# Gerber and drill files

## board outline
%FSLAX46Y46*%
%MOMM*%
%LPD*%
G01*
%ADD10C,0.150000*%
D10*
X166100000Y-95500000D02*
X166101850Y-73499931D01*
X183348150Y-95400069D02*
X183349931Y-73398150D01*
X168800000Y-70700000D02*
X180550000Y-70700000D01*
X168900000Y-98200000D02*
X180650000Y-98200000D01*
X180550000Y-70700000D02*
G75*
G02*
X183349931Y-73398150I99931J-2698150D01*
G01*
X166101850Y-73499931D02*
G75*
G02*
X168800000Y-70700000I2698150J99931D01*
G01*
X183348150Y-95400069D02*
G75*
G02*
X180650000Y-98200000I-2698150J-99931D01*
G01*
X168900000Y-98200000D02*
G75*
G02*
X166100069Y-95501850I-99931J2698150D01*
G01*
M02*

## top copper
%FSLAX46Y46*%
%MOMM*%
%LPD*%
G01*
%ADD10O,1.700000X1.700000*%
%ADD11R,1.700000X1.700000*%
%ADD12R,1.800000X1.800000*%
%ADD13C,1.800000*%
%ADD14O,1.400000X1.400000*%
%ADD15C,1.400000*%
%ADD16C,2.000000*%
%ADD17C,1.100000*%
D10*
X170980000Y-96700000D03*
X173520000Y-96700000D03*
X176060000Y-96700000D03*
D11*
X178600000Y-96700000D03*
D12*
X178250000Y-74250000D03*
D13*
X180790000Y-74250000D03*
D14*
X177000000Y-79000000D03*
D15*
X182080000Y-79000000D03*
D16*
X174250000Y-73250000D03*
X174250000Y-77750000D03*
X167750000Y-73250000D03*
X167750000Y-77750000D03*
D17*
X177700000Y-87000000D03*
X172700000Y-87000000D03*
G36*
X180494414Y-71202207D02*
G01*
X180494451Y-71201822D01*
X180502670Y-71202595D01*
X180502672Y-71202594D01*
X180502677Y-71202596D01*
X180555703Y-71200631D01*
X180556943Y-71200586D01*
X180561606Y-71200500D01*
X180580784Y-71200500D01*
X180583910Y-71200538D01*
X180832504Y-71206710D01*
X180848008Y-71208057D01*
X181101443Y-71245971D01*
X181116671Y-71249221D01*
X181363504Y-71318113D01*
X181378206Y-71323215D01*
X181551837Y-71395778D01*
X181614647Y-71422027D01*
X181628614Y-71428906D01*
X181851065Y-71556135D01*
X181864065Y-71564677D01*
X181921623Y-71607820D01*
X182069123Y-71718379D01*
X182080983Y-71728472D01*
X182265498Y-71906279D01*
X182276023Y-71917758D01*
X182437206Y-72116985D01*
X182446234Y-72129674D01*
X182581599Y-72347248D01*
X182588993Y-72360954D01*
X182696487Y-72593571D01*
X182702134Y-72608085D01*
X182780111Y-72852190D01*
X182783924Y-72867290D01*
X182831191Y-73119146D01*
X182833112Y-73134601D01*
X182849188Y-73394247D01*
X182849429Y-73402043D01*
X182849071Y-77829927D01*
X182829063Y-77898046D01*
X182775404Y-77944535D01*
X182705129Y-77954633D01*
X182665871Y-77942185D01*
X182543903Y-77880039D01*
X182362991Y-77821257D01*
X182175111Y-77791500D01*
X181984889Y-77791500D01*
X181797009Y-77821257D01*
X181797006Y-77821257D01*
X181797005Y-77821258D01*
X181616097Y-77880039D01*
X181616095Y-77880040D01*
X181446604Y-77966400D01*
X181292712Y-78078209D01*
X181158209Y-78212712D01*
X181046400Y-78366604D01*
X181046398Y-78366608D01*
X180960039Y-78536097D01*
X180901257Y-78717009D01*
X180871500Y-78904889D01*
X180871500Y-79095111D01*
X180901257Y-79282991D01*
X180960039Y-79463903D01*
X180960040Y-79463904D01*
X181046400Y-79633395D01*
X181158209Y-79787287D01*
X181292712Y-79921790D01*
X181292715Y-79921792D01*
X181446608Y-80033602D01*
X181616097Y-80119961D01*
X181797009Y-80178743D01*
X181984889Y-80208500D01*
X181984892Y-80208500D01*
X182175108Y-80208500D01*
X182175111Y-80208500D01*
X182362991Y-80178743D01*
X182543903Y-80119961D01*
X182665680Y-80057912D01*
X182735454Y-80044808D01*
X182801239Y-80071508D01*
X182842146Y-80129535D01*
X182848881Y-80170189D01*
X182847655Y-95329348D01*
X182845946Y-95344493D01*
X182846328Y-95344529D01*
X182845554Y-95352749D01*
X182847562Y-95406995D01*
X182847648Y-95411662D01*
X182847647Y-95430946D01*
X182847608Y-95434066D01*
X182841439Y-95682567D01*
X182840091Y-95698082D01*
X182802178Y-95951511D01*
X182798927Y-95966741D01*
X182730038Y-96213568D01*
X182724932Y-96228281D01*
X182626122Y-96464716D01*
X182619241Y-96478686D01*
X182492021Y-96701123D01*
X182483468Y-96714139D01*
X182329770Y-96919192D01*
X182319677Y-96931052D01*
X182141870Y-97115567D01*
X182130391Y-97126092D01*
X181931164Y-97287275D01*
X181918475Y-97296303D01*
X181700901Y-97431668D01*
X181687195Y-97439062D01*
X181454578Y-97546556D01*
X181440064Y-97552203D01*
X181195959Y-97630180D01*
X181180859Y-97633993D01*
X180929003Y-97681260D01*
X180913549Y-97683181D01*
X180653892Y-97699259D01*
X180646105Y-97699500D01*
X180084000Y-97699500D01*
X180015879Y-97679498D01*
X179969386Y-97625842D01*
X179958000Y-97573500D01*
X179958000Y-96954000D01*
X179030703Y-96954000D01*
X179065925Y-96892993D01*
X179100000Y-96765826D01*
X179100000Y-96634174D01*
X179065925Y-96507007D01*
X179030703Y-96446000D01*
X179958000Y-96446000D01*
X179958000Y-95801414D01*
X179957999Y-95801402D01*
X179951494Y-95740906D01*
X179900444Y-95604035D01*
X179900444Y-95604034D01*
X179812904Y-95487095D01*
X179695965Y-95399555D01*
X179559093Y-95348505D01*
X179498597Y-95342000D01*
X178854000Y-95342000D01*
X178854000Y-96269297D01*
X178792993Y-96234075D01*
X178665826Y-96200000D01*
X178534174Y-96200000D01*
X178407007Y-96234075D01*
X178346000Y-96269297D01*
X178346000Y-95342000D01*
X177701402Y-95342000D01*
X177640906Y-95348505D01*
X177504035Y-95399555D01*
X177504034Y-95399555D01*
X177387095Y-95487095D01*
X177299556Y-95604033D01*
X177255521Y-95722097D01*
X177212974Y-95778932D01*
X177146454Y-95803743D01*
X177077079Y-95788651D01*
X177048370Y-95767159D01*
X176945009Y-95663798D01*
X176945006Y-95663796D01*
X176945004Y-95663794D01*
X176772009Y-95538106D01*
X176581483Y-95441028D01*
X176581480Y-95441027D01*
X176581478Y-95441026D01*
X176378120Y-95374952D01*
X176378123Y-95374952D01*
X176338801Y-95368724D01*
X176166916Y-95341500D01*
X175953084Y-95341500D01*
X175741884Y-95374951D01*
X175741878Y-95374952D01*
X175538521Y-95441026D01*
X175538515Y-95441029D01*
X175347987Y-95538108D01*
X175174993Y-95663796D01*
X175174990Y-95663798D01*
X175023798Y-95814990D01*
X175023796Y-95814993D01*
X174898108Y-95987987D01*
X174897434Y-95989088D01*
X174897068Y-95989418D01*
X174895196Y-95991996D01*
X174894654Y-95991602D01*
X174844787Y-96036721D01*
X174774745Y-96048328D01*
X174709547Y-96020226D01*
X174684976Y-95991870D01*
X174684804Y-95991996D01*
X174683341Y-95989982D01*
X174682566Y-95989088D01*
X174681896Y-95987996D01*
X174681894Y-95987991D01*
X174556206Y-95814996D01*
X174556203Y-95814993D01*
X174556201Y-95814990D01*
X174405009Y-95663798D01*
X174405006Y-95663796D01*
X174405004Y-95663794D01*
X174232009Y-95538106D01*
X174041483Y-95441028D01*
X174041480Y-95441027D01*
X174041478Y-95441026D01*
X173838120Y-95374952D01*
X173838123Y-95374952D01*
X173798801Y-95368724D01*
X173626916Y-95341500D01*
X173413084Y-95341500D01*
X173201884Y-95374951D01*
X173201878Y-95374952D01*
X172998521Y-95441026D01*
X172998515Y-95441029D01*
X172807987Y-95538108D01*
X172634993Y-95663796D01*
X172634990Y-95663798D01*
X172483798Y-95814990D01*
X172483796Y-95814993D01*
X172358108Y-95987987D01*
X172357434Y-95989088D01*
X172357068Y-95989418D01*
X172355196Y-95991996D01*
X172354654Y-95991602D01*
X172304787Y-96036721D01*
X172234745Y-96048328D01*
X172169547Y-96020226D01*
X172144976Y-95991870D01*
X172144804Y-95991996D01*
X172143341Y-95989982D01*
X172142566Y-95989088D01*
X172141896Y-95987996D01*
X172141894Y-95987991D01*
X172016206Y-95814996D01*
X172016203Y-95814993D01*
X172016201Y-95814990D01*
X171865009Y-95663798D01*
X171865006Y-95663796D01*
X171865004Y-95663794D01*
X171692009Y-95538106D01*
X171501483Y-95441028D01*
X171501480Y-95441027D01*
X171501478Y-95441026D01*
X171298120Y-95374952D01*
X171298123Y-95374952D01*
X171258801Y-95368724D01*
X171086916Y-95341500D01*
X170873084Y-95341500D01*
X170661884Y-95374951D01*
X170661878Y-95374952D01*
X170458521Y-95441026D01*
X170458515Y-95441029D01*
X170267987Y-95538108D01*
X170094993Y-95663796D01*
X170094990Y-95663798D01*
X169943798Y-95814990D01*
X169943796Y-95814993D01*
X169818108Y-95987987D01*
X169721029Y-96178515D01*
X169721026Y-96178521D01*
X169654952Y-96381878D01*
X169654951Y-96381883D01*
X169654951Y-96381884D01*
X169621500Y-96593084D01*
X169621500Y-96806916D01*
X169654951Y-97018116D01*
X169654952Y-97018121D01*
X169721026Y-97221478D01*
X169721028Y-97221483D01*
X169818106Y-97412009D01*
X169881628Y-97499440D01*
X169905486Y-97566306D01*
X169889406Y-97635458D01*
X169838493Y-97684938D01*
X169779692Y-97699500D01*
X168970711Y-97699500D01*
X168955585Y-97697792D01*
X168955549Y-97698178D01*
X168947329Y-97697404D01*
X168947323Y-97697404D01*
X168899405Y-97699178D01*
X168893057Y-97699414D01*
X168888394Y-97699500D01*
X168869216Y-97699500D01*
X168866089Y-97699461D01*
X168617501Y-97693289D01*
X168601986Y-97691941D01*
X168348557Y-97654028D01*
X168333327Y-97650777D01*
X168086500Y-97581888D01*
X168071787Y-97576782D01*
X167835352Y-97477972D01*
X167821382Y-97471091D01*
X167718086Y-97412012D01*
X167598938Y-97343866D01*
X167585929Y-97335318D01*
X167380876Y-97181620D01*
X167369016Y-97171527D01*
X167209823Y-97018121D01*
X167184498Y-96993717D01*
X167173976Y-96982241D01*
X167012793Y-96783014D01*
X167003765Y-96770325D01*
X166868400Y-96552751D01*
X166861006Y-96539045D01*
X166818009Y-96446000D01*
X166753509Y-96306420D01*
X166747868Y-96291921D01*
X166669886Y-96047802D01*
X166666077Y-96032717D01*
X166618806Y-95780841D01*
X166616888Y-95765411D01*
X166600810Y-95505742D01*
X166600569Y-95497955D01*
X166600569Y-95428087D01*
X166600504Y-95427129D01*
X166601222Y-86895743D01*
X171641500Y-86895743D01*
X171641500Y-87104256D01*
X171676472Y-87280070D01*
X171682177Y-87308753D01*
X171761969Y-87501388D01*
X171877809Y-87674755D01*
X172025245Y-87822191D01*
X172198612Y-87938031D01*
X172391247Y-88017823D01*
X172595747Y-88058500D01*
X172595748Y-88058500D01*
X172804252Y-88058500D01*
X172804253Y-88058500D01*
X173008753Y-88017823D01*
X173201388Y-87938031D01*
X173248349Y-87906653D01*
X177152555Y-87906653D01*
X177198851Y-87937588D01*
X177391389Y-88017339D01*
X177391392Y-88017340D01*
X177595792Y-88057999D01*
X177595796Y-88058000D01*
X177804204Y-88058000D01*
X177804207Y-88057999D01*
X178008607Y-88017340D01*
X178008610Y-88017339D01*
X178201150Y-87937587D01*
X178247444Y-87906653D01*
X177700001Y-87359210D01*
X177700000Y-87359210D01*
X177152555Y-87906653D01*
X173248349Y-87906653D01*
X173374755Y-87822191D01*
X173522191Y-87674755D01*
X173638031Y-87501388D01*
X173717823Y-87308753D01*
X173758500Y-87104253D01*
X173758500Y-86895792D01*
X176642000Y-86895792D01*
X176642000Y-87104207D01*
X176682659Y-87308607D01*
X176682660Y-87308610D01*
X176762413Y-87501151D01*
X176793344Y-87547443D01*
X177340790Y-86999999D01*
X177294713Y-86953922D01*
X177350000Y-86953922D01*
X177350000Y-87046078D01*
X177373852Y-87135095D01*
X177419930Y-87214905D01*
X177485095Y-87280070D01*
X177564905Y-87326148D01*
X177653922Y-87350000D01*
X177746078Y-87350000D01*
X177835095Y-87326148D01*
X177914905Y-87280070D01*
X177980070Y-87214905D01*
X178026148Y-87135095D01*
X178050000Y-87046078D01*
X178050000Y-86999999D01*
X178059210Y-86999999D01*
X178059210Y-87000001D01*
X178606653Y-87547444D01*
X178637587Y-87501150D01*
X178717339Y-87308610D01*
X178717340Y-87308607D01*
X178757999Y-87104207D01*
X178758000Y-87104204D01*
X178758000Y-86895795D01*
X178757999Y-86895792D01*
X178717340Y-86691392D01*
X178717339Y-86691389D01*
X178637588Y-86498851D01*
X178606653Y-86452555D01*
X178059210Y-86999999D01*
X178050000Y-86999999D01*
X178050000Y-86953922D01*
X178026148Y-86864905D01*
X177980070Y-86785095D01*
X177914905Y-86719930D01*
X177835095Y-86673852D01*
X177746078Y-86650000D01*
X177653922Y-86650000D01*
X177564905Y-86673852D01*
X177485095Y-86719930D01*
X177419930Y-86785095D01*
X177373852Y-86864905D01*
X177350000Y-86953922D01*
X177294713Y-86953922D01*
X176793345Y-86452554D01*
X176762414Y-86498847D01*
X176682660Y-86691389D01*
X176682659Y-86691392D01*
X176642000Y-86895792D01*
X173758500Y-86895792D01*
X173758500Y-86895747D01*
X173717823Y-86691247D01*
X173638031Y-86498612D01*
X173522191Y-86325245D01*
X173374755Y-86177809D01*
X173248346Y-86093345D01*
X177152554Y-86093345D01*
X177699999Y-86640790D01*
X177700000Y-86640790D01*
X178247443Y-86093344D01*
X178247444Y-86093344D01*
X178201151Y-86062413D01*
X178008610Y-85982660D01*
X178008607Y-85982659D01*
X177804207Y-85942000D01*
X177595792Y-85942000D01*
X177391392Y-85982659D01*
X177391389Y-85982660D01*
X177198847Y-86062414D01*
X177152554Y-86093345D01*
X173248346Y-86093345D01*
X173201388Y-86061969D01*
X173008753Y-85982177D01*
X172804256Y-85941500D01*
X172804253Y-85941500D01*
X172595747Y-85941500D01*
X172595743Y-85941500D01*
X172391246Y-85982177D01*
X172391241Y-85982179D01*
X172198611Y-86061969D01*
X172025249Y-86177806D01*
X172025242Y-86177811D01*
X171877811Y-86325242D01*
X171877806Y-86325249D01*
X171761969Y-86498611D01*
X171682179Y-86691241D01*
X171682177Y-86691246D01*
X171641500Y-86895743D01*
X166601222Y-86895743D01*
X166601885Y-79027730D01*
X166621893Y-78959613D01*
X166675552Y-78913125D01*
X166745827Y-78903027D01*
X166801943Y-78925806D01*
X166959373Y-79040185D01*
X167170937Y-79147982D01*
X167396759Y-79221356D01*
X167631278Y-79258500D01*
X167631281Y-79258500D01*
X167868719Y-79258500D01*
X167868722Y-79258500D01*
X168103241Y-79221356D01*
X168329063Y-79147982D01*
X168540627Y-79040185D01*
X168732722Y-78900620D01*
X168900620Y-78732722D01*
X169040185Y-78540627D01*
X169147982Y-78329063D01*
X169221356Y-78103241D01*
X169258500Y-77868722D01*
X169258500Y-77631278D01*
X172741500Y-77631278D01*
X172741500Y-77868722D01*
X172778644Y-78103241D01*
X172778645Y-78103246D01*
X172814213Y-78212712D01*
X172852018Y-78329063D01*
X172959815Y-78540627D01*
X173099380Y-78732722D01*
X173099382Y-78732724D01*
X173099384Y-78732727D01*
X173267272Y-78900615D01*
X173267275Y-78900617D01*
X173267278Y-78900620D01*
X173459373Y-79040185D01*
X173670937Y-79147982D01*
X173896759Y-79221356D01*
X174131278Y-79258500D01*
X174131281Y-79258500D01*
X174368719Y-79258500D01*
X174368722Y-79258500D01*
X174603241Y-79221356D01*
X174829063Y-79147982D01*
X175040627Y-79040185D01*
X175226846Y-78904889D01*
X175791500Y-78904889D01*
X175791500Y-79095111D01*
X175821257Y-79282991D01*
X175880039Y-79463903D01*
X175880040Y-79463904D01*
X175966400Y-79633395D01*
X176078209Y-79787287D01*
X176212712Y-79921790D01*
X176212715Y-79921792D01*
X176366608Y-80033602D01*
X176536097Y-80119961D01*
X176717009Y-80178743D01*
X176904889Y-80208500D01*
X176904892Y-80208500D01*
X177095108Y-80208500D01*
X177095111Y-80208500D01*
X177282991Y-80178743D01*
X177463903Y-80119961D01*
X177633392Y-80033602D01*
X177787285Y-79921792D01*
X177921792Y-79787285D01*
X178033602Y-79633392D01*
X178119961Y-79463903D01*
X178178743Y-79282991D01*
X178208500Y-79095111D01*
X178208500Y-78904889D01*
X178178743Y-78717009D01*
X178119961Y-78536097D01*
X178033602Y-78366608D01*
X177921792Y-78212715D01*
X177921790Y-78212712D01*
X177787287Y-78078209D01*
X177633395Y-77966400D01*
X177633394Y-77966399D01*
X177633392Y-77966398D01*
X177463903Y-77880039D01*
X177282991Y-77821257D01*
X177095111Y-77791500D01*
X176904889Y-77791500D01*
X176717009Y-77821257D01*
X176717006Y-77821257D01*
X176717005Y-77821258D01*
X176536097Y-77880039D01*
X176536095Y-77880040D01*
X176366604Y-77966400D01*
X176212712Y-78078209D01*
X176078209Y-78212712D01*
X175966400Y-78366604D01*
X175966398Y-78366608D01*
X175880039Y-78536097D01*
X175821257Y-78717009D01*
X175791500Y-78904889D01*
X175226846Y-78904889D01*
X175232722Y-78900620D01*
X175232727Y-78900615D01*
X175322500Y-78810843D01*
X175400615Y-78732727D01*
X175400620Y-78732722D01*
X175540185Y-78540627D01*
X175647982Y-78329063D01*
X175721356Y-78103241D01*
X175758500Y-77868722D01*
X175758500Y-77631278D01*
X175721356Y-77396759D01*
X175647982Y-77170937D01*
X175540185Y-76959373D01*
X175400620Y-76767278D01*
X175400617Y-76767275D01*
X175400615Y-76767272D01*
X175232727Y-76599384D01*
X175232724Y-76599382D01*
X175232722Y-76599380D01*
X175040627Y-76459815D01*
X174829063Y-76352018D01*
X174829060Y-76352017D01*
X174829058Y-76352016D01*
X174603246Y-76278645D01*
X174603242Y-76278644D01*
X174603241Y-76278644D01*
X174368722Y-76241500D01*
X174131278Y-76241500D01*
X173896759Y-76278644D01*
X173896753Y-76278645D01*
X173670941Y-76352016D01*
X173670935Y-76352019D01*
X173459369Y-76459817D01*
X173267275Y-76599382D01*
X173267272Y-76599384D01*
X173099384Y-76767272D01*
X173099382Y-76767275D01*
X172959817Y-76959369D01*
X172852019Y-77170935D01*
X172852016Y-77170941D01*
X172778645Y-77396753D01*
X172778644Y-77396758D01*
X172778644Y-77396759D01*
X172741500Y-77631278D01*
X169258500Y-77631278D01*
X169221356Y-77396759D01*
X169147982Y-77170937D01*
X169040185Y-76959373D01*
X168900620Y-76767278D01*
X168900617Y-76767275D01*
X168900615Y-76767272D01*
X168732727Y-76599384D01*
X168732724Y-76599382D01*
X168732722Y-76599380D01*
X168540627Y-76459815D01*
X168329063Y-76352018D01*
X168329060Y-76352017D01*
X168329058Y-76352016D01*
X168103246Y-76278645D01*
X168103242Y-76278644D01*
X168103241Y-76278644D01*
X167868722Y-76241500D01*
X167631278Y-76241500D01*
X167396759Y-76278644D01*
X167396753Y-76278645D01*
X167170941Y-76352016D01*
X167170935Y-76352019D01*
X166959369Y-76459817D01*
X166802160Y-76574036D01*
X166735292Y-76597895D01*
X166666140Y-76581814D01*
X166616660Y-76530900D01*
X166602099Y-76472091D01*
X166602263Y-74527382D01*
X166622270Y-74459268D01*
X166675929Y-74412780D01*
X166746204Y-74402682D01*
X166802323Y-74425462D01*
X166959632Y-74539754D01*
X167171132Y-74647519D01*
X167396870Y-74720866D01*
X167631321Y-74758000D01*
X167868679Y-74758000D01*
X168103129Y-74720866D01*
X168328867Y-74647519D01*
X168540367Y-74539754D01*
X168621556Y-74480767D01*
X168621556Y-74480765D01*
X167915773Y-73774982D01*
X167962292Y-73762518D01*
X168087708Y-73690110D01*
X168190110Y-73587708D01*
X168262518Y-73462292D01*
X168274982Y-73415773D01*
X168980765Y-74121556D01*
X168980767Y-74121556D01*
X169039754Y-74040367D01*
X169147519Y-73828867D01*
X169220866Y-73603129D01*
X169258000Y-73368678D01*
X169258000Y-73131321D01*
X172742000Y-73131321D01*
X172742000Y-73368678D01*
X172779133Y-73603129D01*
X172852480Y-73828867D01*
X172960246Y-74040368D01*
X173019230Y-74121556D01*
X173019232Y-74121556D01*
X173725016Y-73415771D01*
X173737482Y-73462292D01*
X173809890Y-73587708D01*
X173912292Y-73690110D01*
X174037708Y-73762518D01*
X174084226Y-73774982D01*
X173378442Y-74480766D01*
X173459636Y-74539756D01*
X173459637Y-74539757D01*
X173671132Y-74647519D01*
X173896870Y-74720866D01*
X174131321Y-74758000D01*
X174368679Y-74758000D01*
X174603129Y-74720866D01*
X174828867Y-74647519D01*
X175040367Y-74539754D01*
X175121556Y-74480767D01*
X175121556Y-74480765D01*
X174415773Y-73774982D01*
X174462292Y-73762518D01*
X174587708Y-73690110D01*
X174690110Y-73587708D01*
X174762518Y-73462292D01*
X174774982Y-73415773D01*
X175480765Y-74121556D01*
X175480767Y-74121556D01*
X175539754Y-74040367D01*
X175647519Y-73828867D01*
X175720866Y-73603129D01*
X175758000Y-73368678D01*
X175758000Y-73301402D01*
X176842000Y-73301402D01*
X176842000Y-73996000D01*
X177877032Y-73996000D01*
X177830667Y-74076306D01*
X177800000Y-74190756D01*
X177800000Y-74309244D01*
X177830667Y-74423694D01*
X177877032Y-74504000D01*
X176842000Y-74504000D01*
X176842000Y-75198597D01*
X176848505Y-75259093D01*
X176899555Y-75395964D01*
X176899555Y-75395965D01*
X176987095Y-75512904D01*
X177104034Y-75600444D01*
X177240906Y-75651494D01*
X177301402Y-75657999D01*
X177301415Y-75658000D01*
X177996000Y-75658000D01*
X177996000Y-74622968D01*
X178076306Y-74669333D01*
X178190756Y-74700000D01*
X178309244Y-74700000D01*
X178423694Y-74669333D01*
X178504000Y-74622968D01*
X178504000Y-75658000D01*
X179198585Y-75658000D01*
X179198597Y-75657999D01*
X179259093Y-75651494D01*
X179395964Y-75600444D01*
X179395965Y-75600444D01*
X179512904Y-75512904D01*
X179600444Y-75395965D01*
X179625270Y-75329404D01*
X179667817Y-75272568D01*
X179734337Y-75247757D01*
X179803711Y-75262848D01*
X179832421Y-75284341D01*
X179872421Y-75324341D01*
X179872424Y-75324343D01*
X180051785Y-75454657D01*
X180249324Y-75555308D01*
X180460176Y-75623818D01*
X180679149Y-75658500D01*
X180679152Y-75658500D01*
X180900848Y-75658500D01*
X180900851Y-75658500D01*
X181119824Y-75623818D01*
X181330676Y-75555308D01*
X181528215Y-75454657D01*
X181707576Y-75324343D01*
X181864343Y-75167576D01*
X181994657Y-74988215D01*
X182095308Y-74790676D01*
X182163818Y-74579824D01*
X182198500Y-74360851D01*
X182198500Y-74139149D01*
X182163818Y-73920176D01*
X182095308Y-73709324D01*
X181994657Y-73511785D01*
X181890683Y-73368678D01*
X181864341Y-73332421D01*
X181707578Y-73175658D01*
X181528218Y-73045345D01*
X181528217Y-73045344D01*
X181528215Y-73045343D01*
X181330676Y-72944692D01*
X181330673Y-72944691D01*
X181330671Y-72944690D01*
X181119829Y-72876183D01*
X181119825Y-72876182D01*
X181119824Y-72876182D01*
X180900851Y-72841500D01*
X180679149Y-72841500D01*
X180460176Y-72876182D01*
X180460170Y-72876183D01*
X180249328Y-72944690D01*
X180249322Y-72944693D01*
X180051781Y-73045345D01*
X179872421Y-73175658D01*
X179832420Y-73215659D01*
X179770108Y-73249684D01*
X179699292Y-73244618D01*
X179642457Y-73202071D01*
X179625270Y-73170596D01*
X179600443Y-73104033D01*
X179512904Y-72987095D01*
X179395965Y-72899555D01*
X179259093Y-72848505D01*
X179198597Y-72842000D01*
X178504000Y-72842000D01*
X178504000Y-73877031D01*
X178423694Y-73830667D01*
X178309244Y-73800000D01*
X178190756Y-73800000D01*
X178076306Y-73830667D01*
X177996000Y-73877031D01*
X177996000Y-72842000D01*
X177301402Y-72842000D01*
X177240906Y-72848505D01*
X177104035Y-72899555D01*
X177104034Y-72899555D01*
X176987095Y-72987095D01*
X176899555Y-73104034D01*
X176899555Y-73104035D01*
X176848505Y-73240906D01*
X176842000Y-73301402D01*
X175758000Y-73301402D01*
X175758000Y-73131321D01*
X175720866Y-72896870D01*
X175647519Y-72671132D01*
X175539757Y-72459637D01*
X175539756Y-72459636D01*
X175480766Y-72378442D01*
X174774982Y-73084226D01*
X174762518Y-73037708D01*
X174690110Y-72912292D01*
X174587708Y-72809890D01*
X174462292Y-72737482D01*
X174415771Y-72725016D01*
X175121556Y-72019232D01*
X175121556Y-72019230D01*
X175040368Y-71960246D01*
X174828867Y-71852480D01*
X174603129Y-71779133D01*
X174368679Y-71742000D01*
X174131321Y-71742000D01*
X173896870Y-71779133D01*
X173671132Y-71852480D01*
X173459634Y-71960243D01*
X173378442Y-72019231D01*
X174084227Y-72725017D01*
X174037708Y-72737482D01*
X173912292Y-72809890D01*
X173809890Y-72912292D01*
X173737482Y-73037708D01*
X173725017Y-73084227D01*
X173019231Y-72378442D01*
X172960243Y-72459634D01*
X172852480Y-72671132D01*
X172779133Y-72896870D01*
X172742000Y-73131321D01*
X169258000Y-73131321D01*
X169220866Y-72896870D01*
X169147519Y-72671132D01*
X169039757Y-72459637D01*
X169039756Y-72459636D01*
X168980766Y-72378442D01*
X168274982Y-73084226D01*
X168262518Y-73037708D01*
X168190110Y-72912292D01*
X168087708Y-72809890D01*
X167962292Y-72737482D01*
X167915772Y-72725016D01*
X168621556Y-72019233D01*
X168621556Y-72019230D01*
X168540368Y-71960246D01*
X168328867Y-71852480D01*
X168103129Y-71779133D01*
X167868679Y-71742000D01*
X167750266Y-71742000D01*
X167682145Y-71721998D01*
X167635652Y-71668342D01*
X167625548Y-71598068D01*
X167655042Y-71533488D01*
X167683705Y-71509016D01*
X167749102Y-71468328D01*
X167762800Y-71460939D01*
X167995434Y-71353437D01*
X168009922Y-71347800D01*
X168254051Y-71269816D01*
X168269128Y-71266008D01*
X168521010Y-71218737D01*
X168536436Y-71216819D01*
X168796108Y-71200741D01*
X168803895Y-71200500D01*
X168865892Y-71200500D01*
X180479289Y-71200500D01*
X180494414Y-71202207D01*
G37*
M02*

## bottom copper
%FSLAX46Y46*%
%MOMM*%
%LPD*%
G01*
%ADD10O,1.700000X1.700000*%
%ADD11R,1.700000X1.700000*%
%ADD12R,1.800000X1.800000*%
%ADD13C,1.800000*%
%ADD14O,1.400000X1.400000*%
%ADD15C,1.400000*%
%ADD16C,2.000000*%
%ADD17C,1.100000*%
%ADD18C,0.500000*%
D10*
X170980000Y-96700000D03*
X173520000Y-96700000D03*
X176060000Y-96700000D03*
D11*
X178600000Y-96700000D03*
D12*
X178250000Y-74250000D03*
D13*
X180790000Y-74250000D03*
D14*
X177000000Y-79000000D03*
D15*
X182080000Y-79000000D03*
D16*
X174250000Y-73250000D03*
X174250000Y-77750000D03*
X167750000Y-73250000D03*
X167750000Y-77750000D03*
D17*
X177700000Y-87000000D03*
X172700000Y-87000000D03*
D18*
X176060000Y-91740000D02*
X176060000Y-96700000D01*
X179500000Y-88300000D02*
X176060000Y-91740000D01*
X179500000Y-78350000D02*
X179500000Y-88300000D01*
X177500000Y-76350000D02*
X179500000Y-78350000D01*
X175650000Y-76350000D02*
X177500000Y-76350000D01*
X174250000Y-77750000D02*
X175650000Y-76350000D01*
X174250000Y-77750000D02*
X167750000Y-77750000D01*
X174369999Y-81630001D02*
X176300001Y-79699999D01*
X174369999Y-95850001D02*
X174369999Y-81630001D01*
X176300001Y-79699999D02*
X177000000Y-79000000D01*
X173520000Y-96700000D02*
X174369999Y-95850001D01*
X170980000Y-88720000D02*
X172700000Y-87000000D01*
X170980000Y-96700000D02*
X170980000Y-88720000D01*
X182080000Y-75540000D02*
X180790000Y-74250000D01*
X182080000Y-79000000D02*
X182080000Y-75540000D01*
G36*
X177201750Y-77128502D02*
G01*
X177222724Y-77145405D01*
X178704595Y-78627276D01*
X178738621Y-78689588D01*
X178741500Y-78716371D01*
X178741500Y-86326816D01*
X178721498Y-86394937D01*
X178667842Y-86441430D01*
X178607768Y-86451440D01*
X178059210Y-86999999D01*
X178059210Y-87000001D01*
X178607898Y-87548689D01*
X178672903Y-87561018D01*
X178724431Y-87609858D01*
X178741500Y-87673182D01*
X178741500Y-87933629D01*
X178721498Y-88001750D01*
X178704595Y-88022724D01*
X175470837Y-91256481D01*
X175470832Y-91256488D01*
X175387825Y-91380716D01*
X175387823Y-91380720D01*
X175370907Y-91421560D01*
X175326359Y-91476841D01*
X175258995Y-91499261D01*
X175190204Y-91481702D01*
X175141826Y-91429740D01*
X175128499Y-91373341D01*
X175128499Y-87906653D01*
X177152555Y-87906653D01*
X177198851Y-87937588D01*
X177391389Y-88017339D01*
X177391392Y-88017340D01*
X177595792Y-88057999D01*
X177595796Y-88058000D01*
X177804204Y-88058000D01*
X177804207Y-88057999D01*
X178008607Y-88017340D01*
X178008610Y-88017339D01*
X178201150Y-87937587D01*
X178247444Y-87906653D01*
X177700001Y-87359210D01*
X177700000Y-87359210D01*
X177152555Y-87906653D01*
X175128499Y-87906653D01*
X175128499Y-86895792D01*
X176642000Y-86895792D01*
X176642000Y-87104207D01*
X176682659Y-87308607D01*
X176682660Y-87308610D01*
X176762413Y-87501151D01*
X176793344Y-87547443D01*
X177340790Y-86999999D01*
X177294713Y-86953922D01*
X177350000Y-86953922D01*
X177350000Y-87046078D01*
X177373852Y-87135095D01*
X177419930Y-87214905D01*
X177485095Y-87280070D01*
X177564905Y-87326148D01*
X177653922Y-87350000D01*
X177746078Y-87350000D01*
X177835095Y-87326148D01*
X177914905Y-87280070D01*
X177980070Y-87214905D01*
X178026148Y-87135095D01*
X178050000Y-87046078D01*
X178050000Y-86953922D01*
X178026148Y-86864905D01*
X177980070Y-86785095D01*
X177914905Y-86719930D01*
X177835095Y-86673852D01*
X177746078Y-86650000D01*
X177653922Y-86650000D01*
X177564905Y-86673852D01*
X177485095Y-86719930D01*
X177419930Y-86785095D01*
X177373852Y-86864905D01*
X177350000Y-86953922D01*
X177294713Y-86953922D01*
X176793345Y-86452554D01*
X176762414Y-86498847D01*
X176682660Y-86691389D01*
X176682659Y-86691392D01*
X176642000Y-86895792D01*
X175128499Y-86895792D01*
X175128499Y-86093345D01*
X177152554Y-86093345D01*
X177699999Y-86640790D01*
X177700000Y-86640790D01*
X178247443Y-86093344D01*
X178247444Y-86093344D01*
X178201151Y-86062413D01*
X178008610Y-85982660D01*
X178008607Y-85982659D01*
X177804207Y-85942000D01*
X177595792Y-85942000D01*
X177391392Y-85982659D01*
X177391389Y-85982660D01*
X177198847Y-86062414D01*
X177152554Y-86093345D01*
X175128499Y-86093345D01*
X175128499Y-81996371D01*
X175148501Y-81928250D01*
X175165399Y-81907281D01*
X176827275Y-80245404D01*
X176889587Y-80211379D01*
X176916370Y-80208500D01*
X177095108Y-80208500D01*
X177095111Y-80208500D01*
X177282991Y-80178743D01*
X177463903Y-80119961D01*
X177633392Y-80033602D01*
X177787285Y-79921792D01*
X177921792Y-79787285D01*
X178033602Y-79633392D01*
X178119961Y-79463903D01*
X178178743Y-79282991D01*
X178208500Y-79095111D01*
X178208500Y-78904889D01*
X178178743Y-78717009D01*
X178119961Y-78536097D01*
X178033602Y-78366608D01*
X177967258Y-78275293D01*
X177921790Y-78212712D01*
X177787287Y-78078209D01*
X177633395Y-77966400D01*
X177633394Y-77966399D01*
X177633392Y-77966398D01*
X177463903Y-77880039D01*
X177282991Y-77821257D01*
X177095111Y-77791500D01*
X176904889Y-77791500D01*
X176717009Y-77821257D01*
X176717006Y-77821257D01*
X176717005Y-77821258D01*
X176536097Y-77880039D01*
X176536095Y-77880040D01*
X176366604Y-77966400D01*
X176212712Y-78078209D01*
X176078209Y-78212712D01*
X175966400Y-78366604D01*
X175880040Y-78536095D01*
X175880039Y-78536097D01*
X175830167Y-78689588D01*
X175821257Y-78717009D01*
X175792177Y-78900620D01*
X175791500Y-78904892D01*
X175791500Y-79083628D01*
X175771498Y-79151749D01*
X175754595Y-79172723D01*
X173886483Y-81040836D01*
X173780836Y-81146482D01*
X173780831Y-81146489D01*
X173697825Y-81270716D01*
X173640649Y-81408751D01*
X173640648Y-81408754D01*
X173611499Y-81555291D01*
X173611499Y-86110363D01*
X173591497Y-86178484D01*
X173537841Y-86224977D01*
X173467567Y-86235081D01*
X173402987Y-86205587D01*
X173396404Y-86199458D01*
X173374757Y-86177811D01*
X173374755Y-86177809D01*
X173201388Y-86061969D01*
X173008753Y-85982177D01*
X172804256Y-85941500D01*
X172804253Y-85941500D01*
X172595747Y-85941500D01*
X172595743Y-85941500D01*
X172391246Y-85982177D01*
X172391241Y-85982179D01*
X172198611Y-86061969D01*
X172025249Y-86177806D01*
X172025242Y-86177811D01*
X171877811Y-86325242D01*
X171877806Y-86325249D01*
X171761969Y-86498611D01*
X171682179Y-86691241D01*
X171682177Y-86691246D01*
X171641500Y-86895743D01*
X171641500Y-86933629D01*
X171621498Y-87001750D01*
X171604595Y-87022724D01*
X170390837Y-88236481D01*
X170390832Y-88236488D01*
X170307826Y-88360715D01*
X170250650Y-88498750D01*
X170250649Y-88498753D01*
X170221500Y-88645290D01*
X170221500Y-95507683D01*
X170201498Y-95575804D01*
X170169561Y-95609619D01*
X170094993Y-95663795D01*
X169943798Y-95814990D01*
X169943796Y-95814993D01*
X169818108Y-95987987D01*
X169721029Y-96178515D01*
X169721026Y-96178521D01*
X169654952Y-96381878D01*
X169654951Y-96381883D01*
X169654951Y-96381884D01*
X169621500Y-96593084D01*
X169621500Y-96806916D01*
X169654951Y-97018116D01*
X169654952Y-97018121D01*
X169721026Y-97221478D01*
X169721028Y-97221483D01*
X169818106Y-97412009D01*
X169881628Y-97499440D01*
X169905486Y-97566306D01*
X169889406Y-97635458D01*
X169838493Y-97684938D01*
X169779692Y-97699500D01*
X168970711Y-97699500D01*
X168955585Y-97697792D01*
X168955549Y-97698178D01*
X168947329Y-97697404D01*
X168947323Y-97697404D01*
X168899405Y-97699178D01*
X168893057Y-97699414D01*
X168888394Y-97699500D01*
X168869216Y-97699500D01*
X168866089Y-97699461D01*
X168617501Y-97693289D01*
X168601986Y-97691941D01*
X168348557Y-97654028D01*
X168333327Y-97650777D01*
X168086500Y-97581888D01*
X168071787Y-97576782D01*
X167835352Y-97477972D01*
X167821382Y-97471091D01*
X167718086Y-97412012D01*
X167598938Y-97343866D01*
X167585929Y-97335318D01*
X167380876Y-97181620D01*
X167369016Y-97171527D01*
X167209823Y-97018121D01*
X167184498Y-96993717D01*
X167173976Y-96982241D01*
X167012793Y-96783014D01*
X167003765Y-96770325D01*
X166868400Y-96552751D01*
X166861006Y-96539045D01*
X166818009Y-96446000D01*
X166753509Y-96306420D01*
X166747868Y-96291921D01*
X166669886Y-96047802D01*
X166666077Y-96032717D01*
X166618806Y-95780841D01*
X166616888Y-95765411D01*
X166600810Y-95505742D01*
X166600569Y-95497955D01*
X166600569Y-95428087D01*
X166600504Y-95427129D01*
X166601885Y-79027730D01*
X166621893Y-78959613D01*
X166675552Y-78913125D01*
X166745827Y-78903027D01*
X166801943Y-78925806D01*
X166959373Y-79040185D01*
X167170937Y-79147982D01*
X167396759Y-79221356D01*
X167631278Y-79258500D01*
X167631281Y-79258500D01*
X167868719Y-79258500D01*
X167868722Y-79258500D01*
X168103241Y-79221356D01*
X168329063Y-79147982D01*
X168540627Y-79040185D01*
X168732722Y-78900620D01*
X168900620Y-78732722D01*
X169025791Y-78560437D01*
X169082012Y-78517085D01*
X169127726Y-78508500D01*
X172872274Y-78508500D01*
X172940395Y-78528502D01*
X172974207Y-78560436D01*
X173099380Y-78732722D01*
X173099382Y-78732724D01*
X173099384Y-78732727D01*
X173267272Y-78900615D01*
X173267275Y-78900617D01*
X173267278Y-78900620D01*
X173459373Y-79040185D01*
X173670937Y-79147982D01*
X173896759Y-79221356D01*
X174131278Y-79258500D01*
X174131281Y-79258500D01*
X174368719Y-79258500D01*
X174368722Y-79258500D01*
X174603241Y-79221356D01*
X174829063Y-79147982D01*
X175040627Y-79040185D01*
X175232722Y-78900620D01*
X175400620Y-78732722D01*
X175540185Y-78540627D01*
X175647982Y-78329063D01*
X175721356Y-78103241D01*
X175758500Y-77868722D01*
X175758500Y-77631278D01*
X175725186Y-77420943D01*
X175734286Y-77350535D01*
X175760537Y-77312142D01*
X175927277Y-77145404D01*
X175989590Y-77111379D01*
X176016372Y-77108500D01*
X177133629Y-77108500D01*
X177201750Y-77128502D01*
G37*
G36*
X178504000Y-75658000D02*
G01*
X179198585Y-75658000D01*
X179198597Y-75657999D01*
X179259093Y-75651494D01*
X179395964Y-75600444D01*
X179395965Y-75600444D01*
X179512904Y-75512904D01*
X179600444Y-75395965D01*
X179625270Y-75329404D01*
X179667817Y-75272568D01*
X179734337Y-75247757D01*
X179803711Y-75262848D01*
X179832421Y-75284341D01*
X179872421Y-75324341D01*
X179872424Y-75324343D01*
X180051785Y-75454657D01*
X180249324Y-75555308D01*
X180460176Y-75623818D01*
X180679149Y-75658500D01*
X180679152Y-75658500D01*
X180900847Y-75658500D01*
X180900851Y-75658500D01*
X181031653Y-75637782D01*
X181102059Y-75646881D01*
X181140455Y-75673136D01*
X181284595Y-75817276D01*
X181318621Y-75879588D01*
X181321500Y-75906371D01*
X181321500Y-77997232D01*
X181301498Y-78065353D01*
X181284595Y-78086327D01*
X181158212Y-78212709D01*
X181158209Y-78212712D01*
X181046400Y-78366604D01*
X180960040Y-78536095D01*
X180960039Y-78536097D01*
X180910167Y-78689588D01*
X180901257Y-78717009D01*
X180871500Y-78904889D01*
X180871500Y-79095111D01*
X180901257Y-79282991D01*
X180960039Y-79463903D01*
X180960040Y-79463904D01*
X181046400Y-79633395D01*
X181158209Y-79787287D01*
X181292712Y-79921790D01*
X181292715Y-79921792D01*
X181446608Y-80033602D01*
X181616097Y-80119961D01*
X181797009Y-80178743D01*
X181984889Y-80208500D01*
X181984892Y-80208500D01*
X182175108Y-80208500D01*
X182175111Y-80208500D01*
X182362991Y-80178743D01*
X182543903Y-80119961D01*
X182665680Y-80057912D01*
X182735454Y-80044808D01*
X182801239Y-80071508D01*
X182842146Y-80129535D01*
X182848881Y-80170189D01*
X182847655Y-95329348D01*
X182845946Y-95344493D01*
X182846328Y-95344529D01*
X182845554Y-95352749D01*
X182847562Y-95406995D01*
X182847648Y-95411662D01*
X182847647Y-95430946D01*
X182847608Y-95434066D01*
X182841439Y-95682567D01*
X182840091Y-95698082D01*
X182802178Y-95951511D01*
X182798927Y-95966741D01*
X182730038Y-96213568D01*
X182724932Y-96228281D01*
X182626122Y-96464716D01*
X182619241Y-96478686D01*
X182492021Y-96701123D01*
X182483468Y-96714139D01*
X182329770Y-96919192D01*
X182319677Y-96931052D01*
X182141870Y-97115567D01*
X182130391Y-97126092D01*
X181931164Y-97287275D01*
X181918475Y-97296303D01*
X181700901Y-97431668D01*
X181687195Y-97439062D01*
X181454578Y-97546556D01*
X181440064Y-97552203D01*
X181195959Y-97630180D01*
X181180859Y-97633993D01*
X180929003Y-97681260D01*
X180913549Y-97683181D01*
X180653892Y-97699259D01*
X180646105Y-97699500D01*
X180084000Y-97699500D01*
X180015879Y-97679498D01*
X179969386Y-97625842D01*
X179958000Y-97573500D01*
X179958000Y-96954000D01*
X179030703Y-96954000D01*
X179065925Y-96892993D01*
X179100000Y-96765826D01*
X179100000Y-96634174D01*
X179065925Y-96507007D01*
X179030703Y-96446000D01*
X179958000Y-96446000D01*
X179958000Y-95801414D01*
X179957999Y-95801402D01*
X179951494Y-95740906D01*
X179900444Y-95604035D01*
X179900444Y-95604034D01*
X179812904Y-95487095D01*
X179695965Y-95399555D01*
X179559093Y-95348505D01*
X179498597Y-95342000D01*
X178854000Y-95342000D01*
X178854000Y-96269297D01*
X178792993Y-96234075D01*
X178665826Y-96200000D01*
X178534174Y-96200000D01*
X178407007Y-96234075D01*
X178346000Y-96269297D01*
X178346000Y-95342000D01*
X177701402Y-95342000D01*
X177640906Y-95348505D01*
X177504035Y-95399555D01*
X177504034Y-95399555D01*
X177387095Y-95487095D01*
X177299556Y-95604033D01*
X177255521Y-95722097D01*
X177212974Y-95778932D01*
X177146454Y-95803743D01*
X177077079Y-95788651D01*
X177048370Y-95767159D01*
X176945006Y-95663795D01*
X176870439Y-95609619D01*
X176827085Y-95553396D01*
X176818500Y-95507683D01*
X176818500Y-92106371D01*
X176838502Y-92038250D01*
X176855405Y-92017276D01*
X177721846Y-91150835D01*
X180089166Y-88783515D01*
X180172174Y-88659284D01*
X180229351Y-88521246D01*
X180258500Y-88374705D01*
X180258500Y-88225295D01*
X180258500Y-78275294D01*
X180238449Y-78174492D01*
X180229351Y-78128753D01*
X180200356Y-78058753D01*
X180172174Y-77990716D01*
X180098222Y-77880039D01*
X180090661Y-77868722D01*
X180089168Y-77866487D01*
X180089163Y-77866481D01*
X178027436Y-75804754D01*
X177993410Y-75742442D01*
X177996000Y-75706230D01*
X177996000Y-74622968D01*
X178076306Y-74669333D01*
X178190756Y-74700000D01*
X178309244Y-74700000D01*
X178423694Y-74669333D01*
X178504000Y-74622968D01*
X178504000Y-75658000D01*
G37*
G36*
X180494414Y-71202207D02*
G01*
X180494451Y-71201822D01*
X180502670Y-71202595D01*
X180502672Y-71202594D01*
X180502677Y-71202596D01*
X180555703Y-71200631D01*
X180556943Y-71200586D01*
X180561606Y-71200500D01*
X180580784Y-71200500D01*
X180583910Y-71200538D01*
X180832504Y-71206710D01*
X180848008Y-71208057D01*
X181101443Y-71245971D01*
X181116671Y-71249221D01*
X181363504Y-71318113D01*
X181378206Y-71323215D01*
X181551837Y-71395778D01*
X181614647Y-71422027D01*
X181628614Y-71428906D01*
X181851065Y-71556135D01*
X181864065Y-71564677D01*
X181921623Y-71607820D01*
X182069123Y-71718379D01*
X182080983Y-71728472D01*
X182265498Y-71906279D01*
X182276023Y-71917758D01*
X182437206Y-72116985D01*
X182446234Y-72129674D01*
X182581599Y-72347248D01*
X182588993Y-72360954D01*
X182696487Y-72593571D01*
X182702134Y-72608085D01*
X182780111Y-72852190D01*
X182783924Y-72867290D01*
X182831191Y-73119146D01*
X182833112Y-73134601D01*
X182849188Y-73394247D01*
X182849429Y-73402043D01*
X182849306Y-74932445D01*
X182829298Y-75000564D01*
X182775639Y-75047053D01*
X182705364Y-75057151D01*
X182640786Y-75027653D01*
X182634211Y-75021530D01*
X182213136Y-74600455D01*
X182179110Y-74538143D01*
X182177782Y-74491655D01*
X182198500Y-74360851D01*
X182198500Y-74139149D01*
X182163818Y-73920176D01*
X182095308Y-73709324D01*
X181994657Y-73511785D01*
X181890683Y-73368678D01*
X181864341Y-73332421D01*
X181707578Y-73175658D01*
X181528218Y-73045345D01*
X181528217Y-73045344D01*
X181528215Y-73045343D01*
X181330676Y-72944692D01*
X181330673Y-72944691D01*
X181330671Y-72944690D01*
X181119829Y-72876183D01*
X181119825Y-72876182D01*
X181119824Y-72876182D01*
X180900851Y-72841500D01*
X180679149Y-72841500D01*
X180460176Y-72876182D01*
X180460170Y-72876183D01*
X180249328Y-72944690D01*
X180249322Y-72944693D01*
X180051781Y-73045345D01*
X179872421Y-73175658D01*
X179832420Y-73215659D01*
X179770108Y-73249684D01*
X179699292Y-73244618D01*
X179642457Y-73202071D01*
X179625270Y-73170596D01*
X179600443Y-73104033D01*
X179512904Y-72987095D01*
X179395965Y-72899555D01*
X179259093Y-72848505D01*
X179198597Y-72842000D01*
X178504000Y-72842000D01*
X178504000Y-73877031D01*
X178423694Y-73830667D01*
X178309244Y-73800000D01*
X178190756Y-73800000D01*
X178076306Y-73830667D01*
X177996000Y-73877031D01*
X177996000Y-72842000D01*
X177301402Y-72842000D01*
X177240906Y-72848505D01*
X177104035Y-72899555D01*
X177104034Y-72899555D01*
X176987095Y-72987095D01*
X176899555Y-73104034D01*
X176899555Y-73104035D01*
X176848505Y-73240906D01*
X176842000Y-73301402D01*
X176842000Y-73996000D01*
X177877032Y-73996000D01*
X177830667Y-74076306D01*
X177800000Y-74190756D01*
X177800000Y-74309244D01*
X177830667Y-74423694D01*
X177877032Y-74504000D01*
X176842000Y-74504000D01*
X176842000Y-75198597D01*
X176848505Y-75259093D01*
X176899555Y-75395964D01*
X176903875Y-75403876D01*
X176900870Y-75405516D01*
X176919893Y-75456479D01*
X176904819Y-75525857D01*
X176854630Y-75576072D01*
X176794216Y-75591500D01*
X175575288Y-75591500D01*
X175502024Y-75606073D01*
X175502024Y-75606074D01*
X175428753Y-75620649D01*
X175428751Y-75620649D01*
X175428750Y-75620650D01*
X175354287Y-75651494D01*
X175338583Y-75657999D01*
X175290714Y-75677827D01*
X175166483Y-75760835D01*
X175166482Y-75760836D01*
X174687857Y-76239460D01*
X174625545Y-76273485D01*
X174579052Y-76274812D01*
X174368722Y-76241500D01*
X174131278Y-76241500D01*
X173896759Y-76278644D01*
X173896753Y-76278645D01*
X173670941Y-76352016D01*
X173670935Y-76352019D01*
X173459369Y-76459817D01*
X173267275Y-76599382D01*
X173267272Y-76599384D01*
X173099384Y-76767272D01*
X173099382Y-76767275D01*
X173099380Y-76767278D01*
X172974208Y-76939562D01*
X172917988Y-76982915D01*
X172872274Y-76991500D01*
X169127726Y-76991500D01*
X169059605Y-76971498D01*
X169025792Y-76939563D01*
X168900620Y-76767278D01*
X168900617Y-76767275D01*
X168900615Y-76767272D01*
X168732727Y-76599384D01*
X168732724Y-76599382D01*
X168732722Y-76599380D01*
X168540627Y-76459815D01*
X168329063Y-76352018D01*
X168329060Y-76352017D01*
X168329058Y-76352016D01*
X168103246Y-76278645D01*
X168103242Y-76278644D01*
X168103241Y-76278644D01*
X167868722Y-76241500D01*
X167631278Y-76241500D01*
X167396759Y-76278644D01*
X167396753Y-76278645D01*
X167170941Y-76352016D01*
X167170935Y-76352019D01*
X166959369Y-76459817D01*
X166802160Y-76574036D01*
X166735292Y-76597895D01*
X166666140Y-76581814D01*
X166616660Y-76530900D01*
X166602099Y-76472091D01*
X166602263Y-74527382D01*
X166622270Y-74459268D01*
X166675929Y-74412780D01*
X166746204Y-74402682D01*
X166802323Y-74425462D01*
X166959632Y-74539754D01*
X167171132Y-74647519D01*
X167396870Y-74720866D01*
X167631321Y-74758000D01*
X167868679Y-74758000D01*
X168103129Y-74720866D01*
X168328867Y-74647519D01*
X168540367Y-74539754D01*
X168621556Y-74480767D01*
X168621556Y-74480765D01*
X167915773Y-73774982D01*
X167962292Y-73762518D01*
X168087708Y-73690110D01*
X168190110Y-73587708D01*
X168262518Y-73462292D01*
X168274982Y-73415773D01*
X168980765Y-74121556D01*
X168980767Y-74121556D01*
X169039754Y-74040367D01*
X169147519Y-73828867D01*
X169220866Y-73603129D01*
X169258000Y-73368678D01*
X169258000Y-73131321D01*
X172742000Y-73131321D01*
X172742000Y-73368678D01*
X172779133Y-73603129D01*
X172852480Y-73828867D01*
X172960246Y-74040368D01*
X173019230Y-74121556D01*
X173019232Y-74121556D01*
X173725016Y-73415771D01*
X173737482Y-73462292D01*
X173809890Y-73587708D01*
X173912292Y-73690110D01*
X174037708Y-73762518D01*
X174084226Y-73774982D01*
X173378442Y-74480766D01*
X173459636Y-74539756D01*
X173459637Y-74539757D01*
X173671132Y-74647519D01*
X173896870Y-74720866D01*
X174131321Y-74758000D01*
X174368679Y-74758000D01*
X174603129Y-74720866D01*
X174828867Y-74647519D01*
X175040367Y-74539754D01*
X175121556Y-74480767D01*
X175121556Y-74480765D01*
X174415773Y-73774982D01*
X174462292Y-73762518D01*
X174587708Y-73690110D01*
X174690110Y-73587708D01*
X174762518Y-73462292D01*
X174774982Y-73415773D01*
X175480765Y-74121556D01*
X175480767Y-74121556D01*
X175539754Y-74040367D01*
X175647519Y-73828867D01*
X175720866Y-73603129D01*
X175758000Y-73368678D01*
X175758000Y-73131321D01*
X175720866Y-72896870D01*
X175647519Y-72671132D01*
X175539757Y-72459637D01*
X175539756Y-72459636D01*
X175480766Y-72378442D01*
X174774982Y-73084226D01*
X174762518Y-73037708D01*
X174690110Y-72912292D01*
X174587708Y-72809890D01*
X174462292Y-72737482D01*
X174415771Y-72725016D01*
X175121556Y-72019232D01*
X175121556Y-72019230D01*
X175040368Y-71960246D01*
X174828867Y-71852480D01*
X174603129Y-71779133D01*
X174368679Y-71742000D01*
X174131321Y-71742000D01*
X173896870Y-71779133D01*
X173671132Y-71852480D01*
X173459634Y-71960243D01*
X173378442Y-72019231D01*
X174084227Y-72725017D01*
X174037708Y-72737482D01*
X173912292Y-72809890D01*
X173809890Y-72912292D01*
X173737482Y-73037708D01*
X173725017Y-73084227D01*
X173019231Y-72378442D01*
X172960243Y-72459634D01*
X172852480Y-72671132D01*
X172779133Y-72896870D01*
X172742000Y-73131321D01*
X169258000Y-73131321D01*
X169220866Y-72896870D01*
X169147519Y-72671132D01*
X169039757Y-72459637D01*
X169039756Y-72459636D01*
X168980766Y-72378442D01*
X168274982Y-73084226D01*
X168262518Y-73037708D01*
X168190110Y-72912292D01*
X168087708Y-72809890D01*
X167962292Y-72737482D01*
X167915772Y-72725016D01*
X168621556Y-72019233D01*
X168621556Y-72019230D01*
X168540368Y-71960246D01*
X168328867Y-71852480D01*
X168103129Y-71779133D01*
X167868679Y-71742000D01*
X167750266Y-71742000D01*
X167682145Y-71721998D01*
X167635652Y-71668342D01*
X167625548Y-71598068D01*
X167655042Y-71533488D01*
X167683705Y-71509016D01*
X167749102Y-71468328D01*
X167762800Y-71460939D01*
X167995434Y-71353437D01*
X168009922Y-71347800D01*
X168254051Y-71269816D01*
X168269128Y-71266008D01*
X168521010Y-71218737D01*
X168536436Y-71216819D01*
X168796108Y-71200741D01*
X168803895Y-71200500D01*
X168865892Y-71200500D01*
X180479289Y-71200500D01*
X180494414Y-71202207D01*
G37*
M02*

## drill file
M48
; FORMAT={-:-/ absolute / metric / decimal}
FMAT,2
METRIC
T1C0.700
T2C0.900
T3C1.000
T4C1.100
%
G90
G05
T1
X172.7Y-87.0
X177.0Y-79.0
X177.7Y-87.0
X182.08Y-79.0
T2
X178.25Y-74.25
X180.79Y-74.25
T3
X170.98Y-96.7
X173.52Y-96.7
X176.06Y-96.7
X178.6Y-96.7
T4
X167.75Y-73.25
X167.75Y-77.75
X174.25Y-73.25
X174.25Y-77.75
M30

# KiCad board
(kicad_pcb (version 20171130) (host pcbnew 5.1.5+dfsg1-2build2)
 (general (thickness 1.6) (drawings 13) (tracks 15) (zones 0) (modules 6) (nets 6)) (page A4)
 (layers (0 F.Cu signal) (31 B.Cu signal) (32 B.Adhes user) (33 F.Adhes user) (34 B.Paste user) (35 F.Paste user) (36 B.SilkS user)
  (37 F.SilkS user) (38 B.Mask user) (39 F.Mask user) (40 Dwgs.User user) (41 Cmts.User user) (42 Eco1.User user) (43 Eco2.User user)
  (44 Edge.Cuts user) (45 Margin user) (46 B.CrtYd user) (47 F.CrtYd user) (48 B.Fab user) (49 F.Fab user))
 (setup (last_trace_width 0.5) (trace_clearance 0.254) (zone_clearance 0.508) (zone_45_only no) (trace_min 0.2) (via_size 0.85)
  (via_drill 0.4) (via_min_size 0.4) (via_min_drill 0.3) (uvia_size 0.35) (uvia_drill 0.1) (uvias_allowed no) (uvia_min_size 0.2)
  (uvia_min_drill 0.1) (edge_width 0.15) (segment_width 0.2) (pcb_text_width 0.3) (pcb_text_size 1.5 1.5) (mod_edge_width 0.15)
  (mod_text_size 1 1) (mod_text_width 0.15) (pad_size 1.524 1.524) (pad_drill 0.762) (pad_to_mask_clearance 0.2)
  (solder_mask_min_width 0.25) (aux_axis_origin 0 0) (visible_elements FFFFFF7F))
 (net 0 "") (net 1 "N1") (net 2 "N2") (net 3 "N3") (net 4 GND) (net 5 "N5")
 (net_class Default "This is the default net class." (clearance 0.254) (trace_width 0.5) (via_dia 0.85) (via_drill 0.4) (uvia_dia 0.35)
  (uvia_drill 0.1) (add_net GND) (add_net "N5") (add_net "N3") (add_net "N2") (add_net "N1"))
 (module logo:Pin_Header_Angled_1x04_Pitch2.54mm (layer F.Cu) (at 178.6 96.7 270)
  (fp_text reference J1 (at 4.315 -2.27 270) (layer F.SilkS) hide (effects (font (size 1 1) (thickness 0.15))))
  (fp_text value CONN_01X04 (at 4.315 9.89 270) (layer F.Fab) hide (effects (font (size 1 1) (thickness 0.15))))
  (pad 4 thru_hole oval (at 0 7.62 270) (size 1.7 1.7) (drill 1) (layers *.Cu *.Mask) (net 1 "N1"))
  (pad 3 thru_hole oval (at 0 5.08 270) (size 1.7 1.7) (drill 1) (layers *.Cu *.Mask) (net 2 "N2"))
  (pad 2 thru_hole oval (at 0 2.54 270) (size 1.7 1.7) (drill 1) (layers *.Cu *.Mask) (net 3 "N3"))
  (pad 1 thru_hole rect (at 0 0 270) (size 1.7 1.7) (drill 1) (layers *.Cu *.Mask) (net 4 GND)))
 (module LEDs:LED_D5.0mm (layer F.Cu) (at 178.25 74.25)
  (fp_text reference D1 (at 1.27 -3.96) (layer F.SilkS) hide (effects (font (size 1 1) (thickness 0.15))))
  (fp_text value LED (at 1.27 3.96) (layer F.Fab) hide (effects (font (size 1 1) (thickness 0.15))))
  (pad 1 thru_hole rect (at 0 0) (size 1.8 1.8) (drill 0.9) (layers *.Cu *.Mask) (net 4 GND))
  (pad 2 thru_hole circle (at 2.54 0) (size 1.8 1.8) (drill 0.9) (layers *.Cu *.Mask) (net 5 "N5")))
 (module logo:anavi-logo (layer F.Cu) (at 167.65 91.1 90)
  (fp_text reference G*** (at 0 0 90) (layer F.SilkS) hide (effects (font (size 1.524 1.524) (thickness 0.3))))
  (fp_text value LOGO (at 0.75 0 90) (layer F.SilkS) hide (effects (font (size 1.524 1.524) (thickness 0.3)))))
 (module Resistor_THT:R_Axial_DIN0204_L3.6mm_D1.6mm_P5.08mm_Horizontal (layer F.Cu) (at 182.08 79 180)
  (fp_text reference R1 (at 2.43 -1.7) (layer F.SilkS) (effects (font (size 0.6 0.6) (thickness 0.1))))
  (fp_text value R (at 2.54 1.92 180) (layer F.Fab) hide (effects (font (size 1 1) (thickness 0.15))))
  (pad 2 thru_hole oval (at 5.08 0 180) (size 1.4 1.4) (drill 0.7) (layers *.Cu *.Mask) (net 2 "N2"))
  (pad 1 thru_hole circle (at 0 0 180) (size 1.4 1.4) (drill 0.7) (layers *.Cu *.Mask) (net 5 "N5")))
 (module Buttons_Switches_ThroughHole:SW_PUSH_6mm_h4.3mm (layer F.Cu) (at 174.25 77.75 180)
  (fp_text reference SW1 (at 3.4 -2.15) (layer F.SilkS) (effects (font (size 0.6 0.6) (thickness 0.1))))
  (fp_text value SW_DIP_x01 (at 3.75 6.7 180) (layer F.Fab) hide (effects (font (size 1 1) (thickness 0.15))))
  (pad 2 thru_hole circle (at 0 4.5 270) (size 2 2) (drill 1.1) (layers *.Cu *.Mask) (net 4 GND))
  (pad 1 thru_hole circle (at 0 0 270) (size 2 2) (drill 1.1) (layers *.Cu *.Mask) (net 3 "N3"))
  (pad 2 thru_hole circle (at 6.5 4.5 270) (size 2 2) (drill 1.1) (layers *.Cu *.Mask) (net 4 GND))
  (pad 1 thru_hole circle (at 6.5 0 270) (size 2 2) (drill 1.1) (layers *.Cu *.Mask) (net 3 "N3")))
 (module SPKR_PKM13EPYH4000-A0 (layer F.Cu) (at 175.2 87 180)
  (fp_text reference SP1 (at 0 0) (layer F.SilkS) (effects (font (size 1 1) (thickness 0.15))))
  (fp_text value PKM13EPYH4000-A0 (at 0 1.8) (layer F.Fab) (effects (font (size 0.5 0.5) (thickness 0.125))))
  (pad N thru_hole circle (at -2.5 0 180) (size 1.1 1.1) (drill 0.7) (layers *.Cu *.Mask) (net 4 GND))
  (pad P thru_hole circle (at 2.5 0 180) (size 1.1 1.1) (drill 0.7) (layers *.Cu *.Mask) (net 1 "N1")))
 (gr_line (start 166.1 95.5) (end 166.10185 73.499931) (layer Edge.Cuts) (width 0.15))
 (gr_line (start 183.34815 95.400069) (end 183.349931 73.39815) (layer Edge.Cuts) (width 0.15))
 (gr_line (start 168.8 70.7) (end 180.55 70.7) (layer Edge.Cuts) (width 0.15))
 (gr_line (start 168.9 98.2) (end 180.65 98.2) (layer Edge.Cuts) (width 0.15))
 (gr_arc (start 180.649931 73.39815) (end 183.349931 73.39815) (angle -92.1210964) (layer Edge.Cuts) (width 0.15))
 (gr_arc (start 168.8 73.4) (end 168.8 70.7) (angle -92.1210964) (layer Edge.Cuts) (width 0.15))
 (gr_arc (start 180.65 95.5) (end 180.65 98.2) (angle -92.1210964) (layer Edge.Cuts) (width 0.15))
 (gr_arc (start 168.800069 95.50185) (end 166.100069 95.50185) (angle -92.1210964) (layer Edge.Cuts) (width 0.15))
 (segment (start 176.06 91.74) (end 176.06 96.7) (width 0.5) (layer B.Cu) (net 3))
 (segment (start 179.5 88.3) (end 176.06 91.74) (width 0.5) (layer B.Cu) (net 3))
 (segment (start 179.5 78.35) (end 179.5 88.3) (width 0.5) (layer B.Cu) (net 3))
 (segment (start 177.5 76.35) (end 179.5 78.35) (width 0.5) (layer B.Cu) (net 3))
 (segment (start 175.65 76.35) (end 177.5 76.35) (width 0.5) (layer B.Cu) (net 3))
 (segment (start 174.25 77.75) (end 175.65 76.35) (width 0.5) (layer B.Cu) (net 3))
 (segment (start 174.25 77.75) (end 167.75 77.75) (width 0.5) (layer B.Cu) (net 3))
 (segment (start 174.369999 81.630001) (end 176.300001 79.699999) (width 0.5) (layer B.Cu) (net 2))
 (segment (start 174.369999 95.850001) (end 174.369999 81.630001) (width 0.5) (layer B.Cu) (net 2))
 (segment (start 176.300001 79.699999) (end 177 79) (width 0.5) (layer B.Cu) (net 2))
 (segment (start 173.52 96.7) (end 174.369999 95.850001) (width 0.5) (layer B.Cu) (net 2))
 (segment (start 170.98 88.72) (end 172.7 87) (width 0.5) (layer B.Cu) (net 1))
 (segment (start 170.98 96.7) (end 170.98 88.72) (width 0.5) (layer B.Cu) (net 1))
 (segment (start 182.08 75.54) (end 180.79 74.25) (width 0.5) (layer B.Cu) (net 5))
 (segment (start 182.08 79) (end 182.08 75.54) (width 0.5) (layer B.Cu) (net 5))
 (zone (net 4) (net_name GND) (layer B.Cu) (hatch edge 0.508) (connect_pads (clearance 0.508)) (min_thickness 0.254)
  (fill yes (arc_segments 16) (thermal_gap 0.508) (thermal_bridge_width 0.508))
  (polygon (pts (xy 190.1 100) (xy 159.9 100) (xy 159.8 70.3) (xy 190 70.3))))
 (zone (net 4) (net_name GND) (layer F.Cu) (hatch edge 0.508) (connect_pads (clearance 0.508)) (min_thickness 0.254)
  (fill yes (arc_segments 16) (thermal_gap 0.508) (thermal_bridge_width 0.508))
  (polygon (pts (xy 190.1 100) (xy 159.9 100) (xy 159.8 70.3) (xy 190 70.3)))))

